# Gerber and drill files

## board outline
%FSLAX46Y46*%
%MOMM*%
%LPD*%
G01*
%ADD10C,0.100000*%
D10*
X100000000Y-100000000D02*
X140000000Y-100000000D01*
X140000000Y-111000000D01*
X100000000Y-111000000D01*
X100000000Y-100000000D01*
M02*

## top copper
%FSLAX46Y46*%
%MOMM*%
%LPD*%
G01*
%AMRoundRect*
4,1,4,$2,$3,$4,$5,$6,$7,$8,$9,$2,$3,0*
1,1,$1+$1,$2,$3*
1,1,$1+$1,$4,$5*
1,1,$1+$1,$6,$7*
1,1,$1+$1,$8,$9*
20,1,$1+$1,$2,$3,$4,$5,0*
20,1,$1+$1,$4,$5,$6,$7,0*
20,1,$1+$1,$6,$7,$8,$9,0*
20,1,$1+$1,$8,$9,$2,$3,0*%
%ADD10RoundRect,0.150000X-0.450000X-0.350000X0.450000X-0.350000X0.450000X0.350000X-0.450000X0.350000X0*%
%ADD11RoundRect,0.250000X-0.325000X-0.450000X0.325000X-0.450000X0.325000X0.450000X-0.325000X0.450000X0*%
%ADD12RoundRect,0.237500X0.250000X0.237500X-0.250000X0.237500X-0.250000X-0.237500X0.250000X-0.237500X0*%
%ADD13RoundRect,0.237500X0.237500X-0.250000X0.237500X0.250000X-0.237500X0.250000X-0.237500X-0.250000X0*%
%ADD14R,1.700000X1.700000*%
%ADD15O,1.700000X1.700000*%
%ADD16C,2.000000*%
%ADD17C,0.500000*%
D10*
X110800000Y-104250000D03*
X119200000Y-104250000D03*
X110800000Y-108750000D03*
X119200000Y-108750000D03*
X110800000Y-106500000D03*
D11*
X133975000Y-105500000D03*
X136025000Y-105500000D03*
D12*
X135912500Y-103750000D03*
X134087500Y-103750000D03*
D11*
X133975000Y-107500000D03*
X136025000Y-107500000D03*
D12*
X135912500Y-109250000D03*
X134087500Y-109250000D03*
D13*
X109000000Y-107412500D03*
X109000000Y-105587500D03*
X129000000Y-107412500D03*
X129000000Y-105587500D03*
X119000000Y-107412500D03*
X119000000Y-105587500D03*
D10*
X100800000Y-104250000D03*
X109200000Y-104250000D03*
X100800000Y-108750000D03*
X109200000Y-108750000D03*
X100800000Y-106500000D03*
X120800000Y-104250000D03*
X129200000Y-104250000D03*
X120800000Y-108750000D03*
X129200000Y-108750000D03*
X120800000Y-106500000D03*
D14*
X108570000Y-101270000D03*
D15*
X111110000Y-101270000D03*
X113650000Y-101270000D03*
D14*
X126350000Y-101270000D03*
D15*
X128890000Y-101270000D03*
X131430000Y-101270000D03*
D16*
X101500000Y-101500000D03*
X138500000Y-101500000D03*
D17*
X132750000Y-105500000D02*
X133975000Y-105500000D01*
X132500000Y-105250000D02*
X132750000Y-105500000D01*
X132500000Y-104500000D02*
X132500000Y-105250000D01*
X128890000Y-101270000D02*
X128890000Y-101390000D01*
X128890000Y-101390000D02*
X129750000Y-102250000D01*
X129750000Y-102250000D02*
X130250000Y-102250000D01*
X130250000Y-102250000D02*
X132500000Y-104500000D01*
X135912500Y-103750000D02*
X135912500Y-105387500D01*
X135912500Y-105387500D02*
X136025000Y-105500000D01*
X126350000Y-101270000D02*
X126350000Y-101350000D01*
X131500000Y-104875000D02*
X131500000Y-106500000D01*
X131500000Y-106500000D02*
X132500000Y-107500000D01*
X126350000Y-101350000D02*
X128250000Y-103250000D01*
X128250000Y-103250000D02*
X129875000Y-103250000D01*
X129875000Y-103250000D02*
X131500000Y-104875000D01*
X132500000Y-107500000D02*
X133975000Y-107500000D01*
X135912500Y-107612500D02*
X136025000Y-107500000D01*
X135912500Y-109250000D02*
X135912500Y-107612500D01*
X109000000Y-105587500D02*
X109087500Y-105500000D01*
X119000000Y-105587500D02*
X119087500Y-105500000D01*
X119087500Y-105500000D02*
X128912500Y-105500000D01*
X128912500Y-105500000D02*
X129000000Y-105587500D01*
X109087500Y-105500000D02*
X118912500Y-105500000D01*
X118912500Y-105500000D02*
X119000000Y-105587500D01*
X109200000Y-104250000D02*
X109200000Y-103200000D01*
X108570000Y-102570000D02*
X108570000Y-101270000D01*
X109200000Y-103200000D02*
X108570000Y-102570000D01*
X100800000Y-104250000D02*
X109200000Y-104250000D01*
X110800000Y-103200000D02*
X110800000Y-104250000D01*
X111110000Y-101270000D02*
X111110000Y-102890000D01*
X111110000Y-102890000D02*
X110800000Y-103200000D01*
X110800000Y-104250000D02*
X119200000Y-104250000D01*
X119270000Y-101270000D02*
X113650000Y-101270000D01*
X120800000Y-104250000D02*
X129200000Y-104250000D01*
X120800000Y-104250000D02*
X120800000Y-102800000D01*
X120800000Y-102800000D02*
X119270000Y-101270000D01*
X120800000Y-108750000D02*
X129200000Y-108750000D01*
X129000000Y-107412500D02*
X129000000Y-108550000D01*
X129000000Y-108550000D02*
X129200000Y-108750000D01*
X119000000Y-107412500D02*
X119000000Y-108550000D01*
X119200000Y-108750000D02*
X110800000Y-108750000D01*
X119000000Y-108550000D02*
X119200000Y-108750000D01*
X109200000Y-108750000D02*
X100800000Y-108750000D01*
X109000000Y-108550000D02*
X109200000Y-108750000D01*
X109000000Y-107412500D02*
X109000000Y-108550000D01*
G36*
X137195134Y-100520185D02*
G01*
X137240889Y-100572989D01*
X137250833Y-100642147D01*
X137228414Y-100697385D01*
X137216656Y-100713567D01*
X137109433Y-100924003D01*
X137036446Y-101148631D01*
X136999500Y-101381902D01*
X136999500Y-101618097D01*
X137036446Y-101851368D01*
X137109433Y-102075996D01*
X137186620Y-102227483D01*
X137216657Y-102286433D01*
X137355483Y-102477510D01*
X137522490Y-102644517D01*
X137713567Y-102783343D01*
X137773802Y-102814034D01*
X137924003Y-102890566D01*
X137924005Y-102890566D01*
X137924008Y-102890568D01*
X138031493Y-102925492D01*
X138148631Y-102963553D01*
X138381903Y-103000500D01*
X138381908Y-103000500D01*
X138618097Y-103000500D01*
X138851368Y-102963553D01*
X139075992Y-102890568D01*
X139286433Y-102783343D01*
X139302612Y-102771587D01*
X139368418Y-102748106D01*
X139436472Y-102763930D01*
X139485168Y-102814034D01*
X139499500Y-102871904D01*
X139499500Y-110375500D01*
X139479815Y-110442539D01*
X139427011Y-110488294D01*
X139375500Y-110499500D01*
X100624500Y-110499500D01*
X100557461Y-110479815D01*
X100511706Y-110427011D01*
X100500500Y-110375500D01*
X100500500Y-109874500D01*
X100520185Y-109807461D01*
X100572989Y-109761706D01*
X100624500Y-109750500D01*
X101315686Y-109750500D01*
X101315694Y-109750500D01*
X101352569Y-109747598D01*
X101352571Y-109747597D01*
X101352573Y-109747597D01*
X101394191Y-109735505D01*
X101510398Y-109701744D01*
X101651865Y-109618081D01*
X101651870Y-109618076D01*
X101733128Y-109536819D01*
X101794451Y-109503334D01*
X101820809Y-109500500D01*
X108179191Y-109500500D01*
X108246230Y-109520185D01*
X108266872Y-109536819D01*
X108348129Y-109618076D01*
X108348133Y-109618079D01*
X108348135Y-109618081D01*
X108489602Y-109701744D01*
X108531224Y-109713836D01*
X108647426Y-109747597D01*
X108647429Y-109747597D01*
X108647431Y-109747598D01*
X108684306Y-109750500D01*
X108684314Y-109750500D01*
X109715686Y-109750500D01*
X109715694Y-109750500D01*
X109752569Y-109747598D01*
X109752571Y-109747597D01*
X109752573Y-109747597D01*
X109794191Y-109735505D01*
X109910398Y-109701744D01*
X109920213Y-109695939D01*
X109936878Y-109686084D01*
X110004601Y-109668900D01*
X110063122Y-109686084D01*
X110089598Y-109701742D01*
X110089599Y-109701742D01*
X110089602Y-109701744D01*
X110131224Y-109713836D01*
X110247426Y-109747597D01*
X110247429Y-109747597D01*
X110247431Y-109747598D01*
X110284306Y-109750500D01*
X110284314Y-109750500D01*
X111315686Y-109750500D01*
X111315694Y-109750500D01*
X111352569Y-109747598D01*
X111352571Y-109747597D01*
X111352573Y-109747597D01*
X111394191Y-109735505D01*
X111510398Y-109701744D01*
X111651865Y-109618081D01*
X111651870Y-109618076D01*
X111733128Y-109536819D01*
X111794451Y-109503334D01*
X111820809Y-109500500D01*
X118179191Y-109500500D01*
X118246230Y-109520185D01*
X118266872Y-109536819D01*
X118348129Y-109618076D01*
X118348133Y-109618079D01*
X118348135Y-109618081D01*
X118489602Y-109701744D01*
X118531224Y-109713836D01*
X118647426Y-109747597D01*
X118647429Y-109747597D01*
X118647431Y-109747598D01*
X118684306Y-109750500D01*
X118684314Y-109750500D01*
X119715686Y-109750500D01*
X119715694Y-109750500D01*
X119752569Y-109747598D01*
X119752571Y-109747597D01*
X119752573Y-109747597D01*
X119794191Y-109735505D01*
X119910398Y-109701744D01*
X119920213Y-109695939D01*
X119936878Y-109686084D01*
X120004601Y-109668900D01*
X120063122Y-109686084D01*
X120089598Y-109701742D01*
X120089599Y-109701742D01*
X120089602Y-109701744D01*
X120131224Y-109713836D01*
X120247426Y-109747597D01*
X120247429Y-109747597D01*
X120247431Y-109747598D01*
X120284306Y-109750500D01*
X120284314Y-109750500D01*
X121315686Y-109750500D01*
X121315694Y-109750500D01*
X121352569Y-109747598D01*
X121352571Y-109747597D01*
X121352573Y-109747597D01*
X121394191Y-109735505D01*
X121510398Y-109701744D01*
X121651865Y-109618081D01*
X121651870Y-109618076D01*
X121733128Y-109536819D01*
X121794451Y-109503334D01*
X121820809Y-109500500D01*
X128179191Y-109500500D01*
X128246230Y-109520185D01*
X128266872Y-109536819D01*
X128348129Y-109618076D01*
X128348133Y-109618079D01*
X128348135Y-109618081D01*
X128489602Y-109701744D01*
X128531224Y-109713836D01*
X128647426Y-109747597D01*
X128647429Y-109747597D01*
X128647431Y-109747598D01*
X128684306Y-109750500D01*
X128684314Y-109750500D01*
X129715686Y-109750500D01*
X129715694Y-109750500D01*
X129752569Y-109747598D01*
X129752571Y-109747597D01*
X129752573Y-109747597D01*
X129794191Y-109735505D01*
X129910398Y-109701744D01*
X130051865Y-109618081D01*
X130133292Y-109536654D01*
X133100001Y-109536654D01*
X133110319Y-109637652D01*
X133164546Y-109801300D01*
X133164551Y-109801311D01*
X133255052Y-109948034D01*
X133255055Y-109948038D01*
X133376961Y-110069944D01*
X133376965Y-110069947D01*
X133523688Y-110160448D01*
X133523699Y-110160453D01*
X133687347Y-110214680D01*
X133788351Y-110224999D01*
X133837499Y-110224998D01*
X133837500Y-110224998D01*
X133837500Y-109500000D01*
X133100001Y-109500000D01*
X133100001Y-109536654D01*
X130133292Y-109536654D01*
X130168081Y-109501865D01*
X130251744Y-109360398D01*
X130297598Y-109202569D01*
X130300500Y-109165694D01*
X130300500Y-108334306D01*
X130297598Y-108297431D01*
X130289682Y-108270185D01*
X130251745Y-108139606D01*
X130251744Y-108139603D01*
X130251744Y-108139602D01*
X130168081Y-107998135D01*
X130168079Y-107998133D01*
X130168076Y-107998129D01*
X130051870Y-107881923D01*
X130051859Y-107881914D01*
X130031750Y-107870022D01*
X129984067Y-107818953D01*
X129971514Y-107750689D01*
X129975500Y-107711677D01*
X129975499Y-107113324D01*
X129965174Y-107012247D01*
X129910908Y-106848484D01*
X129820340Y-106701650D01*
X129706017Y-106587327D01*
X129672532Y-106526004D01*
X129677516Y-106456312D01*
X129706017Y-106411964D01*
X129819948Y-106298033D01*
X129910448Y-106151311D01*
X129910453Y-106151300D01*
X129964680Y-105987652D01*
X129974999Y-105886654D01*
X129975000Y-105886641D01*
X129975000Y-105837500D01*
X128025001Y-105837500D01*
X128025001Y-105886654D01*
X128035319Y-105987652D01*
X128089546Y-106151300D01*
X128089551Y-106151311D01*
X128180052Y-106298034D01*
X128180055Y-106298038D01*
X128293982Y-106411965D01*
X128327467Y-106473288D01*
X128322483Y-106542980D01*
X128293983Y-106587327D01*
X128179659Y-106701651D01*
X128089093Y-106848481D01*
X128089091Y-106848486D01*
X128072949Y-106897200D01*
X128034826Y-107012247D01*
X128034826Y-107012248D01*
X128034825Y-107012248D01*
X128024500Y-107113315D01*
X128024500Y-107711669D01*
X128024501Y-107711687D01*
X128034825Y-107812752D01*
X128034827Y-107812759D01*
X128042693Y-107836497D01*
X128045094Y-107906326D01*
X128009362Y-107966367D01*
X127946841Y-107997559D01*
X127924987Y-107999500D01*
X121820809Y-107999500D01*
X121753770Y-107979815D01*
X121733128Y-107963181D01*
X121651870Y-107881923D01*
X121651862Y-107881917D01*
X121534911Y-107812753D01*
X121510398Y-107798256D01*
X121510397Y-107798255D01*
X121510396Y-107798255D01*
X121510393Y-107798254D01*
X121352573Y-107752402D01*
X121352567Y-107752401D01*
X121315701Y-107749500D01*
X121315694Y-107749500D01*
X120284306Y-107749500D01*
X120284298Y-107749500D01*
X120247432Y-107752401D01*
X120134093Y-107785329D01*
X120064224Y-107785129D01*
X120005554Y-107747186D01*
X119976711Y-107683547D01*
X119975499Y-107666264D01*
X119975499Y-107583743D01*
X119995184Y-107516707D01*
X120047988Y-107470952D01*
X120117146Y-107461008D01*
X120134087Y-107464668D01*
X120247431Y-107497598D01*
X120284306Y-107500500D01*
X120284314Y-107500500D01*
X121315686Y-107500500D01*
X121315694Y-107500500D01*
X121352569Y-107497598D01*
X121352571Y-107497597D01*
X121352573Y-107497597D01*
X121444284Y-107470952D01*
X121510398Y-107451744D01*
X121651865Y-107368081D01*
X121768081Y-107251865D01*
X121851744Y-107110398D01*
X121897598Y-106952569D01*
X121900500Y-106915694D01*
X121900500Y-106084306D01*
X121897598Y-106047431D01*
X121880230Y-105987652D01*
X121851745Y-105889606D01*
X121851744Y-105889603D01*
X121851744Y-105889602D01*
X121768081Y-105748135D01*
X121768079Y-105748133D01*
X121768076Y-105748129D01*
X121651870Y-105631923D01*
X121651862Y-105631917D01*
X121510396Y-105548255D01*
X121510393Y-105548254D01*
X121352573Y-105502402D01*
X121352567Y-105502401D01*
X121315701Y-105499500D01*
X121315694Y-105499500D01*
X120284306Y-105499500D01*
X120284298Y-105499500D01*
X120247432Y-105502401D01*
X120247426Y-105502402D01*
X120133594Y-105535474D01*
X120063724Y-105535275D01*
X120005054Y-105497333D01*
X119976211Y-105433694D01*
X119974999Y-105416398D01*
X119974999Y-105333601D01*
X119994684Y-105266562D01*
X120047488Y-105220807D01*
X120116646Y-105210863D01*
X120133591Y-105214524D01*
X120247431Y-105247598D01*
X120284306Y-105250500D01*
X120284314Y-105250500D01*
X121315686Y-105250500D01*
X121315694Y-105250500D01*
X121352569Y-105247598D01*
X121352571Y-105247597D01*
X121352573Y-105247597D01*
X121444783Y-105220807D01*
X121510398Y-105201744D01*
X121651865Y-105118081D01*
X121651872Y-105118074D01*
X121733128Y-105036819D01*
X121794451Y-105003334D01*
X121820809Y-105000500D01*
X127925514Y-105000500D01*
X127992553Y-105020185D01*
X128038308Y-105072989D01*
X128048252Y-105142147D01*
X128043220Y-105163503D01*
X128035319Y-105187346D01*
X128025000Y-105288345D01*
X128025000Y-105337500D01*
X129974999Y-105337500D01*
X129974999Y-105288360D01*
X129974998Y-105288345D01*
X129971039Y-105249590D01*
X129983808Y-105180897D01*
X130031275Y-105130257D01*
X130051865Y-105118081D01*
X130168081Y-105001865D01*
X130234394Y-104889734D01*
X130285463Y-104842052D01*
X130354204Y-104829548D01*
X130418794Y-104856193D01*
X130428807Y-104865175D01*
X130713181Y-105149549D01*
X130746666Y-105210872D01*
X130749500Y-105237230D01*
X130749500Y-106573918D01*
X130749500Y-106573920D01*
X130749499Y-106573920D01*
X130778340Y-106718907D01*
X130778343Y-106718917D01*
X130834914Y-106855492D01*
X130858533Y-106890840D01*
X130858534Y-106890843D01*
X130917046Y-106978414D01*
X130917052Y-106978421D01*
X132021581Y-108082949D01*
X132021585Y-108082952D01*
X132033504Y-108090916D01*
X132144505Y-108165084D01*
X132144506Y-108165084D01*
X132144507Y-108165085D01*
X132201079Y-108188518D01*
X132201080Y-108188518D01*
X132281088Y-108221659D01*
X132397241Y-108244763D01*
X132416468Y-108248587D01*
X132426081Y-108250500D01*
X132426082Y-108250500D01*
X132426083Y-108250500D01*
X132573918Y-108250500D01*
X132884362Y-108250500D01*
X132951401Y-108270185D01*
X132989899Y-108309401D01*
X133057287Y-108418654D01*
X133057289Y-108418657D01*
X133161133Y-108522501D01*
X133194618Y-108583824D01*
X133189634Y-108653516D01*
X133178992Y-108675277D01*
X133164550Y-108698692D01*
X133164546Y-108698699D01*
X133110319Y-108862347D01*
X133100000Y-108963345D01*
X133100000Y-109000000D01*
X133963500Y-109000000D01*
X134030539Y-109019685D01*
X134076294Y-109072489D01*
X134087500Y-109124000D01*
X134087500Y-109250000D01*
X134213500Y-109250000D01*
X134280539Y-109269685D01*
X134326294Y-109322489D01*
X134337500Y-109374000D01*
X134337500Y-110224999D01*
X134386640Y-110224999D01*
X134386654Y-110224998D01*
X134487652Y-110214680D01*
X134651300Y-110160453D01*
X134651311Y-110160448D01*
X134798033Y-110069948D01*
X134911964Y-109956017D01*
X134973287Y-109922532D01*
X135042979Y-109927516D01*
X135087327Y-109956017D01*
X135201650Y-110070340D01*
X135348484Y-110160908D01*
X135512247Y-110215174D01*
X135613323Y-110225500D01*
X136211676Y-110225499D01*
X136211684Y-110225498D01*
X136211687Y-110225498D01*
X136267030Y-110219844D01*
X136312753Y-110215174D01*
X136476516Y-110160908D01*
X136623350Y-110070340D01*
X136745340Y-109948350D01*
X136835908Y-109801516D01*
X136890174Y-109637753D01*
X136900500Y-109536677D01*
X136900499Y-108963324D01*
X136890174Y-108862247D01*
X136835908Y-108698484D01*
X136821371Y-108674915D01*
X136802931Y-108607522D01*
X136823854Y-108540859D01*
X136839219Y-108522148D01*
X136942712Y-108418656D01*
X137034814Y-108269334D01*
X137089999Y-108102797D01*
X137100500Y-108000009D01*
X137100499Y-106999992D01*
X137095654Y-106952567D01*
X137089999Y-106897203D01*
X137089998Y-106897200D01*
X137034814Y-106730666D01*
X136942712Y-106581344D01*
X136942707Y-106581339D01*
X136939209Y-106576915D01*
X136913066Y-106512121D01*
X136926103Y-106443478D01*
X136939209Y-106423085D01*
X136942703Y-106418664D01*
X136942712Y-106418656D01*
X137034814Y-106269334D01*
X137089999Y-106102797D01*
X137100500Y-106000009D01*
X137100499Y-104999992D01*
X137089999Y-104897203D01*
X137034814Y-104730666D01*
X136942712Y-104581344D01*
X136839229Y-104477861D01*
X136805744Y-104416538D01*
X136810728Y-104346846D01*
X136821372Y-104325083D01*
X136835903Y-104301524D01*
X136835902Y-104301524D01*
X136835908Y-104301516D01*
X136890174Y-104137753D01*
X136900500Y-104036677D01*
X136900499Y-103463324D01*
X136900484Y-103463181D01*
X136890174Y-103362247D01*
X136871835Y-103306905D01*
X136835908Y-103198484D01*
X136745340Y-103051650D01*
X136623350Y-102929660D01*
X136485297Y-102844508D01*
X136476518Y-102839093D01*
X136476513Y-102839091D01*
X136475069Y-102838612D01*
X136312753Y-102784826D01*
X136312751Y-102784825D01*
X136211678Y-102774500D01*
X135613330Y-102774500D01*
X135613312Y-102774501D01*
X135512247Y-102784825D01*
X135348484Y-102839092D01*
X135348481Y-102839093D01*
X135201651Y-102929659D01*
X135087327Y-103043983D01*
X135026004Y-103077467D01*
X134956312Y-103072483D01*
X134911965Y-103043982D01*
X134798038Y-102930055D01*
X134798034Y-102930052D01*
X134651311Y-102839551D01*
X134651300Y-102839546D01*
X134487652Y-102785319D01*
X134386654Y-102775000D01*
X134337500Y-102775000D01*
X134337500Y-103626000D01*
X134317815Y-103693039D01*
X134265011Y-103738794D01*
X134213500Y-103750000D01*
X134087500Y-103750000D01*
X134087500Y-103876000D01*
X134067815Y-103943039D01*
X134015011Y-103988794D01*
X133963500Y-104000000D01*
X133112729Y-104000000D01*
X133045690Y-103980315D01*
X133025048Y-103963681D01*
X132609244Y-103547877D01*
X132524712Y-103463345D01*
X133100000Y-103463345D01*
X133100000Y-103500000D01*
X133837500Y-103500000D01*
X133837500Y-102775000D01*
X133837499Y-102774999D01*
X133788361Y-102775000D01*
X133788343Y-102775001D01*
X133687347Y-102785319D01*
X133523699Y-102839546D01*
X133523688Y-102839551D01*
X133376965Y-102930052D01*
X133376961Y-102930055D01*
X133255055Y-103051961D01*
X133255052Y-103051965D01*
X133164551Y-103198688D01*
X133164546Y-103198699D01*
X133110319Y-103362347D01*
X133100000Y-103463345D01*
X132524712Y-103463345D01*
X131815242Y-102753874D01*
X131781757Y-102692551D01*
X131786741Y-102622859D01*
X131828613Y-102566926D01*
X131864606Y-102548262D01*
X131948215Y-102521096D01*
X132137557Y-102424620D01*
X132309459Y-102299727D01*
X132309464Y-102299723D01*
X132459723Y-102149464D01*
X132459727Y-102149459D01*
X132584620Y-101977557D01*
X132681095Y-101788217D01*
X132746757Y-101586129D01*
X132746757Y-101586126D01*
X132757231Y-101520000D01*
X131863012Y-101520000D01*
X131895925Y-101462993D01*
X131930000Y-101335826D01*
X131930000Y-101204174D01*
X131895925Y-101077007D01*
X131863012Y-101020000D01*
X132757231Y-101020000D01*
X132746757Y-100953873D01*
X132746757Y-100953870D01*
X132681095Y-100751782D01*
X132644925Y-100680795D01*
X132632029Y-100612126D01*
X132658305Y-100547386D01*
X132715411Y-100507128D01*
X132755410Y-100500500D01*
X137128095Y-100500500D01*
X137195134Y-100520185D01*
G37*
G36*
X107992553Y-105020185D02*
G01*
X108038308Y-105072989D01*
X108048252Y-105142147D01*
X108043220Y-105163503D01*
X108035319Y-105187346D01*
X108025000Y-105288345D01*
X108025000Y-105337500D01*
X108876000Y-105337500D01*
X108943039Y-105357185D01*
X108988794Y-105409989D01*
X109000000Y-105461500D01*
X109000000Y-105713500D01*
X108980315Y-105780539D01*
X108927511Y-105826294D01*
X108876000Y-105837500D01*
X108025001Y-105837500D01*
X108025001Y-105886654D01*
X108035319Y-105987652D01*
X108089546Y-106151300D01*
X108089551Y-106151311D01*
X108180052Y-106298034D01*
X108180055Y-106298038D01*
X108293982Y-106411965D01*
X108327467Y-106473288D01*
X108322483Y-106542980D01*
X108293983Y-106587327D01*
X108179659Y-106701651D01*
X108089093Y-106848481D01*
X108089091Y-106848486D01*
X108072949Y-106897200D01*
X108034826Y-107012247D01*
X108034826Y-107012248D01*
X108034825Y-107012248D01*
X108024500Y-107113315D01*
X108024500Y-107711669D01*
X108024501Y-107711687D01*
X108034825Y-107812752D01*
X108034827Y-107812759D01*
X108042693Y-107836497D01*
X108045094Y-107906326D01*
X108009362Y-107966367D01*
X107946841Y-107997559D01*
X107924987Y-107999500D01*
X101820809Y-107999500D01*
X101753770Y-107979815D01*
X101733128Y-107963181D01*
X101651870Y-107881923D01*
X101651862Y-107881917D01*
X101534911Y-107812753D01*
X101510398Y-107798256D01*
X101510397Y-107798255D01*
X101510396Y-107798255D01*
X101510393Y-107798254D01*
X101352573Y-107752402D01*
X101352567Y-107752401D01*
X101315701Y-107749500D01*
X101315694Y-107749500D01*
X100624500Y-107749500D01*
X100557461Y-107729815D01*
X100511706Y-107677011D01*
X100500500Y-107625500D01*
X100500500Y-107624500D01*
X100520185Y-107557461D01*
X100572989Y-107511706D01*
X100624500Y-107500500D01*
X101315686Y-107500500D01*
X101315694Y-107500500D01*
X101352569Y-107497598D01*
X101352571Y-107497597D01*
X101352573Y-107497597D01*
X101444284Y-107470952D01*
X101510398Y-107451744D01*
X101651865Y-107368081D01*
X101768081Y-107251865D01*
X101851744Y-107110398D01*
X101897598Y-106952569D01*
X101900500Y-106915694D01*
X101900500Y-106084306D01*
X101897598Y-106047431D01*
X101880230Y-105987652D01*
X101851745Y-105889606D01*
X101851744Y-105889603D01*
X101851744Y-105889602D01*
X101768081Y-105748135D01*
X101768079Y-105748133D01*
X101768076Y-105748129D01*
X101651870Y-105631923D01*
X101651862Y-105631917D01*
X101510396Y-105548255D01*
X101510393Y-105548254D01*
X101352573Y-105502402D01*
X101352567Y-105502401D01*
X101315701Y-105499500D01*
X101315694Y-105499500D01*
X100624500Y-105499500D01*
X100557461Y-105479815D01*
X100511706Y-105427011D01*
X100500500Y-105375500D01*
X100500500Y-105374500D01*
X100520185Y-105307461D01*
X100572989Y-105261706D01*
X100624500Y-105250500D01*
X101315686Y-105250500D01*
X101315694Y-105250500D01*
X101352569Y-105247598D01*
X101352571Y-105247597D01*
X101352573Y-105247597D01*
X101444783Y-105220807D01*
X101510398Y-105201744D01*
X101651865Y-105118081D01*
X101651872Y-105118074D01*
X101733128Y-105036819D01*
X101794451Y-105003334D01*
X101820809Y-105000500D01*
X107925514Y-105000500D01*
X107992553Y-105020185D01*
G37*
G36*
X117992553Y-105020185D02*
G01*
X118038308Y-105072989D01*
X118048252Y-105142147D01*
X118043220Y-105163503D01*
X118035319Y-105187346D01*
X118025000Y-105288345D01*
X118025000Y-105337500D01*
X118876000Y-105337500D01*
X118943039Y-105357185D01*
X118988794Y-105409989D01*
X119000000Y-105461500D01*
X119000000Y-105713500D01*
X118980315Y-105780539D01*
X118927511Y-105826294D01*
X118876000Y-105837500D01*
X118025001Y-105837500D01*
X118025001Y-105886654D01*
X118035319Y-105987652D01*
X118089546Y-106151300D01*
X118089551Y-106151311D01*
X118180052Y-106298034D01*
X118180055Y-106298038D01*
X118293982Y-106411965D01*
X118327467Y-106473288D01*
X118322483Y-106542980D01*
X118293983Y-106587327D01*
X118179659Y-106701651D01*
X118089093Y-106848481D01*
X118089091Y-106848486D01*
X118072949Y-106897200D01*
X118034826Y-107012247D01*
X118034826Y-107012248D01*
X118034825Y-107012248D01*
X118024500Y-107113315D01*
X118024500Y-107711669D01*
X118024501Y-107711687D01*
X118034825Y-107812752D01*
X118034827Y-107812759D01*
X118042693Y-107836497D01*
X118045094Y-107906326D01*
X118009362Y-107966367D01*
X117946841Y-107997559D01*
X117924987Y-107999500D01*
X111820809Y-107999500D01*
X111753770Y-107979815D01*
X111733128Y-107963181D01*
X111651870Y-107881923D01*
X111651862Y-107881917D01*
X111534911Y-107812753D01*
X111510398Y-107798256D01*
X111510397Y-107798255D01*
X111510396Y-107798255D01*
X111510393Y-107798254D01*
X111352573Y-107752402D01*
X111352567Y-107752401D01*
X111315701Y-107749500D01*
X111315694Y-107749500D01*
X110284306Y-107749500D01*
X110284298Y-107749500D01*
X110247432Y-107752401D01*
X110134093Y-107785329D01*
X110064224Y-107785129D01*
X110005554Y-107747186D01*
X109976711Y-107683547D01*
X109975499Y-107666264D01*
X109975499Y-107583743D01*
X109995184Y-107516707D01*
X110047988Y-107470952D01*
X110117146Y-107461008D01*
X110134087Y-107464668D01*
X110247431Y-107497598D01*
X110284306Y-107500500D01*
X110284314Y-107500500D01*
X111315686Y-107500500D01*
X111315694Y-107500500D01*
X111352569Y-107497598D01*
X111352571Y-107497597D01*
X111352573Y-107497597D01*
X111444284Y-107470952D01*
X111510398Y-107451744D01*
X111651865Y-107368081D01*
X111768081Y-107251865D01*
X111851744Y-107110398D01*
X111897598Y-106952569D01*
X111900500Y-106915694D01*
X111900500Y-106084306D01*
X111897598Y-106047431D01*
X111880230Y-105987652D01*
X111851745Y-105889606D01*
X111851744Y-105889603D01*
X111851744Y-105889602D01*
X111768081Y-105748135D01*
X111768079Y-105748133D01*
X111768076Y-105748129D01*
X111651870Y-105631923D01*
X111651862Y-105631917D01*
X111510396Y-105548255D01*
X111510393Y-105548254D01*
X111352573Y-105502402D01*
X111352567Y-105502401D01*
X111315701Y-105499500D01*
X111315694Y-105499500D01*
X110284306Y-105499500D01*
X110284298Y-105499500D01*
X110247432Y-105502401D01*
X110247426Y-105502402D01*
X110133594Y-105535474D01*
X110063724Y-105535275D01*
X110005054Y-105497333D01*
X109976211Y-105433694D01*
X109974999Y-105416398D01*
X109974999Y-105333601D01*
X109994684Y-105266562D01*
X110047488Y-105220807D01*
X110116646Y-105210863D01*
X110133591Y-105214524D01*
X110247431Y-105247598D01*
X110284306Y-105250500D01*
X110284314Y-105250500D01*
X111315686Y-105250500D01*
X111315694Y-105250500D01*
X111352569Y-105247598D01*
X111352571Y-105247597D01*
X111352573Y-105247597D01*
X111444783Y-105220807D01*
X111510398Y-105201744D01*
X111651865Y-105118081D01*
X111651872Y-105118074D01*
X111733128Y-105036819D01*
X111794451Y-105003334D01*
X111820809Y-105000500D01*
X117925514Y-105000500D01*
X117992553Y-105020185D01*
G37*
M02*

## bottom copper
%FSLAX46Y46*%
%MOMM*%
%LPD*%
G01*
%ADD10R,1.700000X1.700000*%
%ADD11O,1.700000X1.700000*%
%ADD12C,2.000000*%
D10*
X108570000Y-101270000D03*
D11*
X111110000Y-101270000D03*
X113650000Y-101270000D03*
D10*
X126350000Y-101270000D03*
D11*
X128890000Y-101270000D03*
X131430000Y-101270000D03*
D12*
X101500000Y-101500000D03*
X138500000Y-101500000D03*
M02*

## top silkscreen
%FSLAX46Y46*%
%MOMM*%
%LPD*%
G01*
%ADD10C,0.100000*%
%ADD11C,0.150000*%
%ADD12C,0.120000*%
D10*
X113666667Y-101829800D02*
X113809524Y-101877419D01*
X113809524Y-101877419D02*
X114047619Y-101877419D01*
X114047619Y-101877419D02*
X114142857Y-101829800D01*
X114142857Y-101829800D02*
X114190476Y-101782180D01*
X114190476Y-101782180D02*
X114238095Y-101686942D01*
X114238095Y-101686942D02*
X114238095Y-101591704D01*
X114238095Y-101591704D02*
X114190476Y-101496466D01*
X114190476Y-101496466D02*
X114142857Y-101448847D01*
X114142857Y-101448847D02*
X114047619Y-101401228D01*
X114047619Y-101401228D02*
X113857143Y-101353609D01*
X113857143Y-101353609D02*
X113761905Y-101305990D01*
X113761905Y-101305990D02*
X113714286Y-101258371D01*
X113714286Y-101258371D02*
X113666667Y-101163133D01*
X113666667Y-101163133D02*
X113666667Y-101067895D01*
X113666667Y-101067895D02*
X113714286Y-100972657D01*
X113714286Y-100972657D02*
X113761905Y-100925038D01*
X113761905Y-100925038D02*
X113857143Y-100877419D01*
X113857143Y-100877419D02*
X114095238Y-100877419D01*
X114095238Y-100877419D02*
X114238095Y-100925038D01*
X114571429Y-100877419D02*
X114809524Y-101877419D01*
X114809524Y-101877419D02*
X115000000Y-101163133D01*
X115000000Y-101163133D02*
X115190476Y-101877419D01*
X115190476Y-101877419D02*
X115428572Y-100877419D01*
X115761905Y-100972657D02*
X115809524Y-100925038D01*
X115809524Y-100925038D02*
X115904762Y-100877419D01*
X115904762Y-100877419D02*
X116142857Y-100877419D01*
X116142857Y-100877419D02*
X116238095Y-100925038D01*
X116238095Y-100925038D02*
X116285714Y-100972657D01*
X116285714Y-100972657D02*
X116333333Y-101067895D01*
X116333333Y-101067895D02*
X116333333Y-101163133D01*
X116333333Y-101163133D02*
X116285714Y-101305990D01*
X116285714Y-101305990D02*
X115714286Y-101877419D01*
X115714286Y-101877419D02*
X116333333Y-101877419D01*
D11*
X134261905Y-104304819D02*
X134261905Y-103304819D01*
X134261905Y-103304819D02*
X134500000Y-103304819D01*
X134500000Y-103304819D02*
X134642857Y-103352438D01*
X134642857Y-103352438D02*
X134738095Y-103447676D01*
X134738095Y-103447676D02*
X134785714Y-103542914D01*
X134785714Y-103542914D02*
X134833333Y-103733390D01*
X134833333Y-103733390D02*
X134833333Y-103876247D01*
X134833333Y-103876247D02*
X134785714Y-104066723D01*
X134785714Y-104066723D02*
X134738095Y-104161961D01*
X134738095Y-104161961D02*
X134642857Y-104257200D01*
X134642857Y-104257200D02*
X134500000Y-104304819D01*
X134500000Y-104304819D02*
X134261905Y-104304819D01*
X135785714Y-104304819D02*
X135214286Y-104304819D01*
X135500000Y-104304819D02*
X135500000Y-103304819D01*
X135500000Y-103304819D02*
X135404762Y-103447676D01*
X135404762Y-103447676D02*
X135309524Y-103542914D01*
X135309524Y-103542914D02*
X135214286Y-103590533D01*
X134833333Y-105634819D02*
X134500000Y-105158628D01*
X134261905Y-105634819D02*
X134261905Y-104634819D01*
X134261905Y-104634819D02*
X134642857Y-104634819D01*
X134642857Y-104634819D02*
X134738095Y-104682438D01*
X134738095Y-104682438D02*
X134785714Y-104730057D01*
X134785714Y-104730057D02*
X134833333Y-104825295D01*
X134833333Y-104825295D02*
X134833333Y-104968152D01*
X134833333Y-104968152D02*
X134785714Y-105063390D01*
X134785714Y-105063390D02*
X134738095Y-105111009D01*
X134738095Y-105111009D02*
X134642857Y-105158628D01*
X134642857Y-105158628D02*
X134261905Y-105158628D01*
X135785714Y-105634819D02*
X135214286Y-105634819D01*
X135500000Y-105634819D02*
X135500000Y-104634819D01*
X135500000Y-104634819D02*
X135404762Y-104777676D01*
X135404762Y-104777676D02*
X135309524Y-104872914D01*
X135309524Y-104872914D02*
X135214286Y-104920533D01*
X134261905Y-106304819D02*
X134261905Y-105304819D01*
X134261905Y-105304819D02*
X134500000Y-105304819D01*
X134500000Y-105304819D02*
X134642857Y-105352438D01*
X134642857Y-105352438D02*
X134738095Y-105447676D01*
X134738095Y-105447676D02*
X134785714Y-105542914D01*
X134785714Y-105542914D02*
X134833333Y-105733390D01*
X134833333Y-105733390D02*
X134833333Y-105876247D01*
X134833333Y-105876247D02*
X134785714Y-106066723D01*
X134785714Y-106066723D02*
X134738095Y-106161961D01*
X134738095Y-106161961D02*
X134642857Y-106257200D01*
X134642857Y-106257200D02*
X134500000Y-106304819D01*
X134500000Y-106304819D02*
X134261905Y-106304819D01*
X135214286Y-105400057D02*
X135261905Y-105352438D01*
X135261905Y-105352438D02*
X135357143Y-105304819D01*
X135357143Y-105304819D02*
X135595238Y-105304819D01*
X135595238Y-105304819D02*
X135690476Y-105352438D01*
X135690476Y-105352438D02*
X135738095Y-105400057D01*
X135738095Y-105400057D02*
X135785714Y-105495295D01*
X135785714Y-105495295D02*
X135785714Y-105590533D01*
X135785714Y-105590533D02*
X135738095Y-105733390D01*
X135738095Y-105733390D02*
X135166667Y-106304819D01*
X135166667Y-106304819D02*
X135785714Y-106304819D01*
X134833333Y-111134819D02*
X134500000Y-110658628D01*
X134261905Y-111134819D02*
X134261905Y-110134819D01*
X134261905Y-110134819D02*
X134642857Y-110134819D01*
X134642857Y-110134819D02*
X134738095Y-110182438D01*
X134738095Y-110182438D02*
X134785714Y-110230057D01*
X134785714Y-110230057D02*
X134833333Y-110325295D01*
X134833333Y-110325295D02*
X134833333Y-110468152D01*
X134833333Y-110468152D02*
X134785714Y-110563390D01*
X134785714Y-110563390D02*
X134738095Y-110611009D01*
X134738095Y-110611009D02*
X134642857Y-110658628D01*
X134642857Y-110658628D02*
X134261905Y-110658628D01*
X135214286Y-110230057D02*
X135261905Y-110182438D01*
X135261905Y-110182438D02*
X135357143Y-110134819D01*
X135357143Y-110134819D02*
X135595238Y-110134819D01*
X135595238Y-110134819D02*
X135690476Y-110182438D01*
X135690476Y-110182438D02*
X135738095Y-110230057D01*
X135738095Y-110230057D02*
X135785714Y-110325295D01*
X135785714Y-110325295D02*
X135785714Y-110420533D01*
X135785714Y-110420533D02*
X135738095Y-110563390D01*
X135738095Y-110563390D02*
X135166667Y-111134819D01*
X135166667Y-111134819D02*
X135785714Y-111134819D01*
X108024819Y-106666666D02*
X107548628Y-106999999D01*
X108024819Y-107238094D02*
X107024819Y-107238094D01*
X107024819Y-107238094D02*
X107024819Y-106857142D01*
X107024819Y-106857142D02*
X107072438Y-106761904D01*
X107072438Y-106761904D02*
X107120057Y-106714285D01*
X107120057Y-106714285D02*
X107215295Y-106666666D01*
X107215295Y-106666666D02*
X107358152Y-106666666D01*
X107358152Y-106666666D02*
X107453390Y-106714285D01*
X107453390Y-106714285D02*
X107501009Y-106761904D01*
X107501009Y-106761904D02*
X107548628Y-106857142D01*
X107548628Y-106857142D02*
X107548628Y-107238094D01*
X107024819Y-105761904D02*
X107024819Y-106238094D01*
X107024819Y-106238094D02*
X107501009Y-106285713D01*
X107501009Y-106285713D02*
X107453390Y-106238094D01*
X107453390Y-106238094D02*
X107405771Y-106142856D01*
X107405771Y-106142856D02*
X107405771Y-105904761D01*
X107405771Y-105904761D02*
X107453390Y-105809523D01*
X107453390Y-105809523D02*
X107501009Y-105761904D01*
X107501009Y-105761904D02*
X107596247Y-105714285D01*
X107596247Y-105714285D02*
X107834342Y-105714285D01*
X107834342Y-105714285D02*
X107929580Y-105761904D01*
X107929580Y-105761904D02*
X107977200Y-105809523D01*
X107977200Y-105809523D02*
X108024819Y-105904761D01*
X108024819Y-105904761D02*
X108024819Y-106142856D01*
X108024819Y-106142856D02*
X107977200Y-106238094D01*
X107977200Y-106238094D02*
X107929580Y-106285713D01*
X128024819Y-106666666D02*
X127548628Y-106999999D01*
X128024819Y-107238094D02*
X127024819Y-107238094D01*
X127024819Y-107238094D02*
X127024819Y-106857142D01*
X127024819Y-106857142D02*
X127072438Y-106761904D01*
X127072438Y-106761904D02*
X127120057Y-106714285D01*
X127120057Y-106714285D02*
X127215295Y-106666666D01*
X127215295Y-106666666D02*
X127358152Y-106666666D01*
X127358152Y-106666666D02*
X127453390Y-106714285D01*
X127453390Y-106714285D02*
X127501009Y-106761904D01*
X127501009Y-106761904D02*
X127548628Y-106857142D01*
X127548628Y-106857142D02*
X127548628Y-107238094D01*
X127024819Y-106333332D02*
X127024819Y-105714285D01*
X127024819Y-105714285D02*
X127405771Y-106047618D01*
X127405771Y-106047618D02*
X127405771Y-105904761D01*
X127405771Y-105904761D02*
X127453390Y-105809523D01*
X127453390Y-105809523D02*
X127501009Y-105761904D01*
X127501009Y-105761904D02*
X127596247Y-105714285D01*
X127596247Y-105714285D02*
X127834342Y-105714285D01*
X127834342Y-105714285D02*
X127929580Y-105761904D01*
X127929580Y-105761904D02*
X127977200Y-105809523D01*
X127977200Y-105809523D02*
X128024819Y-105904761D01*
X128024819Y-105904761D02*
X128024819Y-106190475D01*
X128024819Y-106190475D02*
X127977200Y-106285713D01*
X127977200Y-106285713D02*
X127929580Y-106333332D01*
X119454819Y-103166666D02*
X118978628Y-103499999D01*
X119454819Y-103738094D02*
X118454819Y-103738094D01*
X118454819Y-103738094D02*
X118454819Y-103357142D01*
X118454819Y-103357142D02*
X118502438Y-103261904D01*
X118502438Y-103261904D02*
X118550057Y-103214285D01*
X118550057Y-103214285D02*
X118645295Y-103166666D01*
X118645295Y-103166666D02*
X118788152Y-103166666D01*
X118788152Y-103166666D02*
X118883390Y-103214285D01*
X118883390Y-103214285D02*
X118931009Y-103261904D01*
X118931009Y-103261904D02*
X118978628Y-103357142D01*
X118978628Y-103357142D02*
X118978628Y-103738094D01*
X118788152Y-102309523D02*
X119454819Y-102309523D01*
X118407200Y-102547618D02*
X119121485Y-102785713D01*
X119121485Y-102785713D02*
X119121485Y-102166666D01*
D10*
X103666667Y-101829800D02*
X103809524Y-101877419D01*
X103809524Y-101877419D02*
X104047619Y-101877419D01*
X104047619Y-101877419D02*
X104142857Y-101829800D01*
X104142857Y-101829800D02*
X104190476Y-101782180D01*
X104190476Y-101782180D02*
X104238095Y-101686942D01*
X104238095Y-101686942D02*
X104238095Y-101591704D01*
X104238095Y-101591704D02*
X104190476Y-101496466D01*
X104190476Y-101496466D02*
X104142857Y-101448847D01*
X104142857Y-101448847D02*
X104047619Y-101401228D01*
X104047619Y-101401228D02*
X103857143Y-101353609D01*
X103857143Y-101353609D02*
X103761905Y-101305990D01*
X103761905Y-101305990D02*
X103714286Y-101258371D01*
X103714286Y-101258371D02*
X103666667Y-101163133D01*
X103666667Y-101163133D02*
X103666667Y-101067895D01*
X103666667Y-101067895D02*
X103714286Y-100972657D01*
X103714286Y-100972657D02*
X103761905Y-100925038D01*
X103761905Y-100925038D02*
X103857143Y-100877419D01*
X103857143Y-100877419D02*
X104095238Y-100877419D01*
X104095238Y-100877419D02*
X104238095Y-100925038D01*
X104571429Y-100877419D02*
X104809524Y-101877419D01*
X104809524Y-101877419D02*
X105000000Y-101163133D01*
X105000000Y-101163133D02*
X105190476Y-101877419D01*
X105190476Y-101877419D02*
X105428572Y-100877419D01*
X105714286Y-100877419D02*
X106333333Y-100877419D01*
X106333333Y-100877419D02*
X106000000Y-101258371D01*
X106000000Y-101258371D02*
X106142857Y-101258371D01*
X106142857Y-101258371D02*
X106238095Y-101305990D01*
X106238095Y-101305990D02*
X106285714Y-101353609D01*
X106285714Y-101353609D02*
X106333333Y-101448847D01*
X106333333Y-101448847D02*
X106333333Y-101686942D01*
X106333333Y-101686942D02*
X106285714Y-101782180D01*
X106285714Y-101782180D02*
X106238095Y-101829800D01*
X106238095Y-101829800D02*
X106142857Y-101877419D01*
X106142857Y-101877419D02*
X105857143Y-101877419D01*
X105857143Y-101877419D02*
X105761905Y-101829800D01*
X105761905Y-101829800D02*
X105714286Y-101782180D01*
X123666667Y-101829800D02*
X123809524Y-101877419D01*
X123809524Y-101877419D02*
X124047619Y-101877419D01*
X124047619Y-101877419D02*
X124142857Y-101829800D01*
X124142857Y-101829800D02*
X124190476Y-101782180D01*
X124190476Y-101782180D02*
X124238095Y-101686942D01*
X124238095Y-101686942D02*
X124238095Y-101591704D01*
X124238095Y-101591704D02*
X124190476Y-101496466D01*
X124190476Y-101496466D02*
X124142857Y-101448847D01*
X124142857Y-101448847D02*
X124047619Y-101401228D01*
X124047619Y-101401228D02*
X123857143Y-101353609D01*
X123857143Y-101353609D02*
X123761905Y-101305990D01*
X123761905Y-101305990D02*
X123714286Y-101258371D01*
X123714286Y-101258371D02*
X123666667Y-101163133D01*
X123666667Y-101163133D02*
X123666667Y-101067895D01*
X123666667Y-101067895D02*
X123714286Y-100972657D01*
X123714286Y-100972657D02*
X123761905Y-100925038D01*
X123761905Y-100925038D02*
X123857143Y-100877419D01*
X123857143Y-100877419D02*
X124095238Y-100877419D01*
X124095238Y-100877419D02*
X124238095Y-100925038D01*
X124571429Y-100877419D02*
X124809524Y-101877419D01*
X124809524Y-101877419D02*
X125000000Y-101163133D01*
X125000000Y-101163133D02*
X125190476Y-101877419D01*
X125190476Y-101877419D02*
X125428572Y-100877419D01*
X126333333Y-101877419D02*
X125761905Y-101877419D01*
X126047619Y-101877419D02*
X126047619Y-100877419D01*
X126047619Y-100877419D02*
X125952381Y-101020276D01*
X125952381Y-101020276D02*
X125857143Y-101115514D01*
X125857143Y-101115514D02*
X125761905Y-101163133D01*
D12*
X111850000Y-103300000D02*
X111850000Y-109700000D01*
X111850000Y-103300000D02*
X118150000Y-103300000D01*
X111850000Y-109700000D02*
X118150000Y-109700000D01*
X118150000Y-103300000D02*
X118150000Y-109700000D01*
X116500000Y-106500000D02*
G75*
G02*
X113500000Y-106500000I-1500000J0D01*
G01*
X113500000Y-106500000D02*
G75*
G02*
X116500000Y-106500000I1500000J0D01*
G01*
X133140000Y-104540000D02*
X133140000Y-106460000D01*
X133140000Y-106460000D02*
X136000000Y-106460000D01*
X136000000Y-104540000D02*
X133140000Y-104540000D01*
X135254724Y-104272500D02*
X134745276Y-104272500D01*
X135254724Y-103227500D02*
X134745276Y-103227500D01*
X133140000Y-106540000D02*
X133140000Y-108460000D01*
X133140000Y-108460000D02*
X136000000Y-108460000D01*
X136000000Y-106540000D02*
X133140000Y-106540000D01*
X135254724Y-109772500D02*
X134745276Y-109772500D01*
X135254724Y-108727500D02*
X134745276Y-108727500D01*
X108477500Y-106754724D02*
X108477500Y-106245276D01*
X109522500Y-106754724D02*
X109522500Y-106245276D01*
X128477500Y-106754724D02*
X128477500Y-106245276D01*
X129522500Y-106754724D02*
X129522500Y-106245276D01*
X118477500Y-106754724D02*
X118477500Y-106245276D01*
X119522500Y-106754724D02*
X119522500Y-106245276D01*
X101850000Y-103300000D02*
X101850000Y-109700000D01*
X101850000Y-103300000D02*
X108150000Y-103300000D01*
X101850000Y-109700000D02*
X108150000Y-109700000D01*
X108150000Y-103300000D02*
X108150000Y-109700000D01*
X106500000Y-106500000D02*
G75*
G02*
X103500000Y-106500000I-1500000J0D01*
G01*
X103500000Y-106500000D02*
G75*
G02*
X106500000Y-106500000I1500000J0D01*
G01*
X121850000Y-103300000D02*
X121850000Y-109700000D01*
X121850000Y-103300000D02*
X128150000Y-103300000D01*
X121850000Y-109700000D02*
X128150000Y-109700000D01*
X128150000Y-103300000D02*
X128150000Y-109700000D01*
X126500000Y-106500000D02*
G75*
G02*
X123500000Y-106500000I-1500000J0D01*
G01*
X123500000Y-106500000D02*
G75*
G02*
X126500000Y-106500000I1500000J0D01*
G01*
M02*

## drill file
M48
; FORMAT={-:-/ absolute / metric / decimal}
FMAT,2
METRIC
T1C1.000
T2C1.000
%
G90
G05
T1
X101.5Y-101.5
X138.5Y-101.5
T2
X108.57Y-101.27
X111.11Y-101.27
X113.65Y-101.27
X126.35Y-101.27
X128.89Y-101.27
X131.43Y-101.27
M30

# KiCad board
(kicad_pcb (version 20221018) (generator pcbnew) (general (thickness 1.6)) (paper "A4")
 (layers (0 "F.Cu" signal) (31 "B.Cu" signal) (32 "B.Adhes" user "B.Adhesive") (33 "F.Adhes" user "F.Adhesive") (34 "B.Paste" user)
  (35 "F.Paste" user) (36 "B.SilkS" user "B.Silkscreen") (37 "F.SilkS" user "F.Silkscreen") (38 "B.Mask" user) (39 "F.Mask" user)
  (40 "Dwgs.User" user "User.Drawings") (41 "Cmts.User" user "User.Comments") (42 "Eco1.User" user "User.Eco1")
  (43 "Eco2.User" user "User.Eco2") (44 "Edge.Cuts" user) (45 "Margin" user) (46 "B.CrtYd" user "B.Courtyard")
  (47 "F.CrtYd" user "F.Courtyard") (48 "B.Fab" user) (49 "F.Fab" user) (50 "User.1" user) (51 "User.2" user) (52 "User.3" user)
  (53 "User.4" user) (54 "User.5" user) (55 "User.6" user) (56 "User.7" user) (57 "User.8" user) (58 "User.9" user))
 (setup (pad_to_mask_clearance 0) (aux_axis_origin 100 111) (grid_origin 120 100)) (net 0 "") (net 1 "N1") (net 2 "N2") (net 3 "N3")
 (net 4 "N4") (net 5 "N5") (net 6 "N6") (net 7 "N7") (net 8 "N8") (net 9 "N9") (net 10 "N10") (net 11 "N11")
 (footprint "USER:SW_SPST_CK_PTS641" (layer "F.Cu") (at 115 106.5)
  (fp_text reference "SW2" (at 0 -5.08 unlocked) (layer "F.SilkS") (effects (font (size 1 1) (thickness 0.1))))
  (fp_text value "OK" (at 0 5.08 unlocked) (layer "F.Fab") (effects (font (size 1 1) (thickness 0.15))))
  (fp_line (start -3.15 -3.2) (end -3.15 3.2) (stroke (width 0.12) (type default)) (layer "F.SilkS"))
  (fp_line (start -3.15 -3.2) (end 3.15 -3.2) (stroke (width 0.12) (type solid)) (layer "F.SilkS"))
  (fp_line (start -3.15 3.2) (end 3.15 3.2) (stroke (width 0.12) (type solid)) (layer "F.SilkS"))
  (fp_line (start 3.15 -3.2) (end 3.15 3.2) (stroke (width 0.12) (type solid)) (layer "F.SilkS"))
  (fp_circle (center 0 0) (end 1.5 0) (stroke (width 0.12) (type default)) (fill none) (layer "F.SilkS"))
  (pad "1" smd roundrect (at -4.2 -2.25) (size 1.2 1) (layers "F.Cu" "F.Paste" "F.Mask") (roundrect_rratio 0.15) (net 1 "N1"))
  (pad "1" smd roundrect (at 4.2 -2.25) (size 1.2 1) (layers "F.Cu" "F.Paste" "F.Mask") (roundrect_rratio 0.15) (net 1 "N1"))
  (pad "2" smd roundrect (at -4.2 2.25) (size 1.2 1) (layers "F.Cu" "F.Paste" "F.Mask") (roundrect_rratio 0.15) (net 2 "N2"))
  (pad "2" smd roundrect (at 4.2 2.25) (size 1.2 1) (layers "F.Cu" "F.Paste" "F.Mask") (roundrect_rratio 0.15) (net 2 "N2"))
  (pad "SH" smd roundrect (at -4.2 0) (size 1.2 1) (layers "F.Cu" "F.Paste" "F.Mask") (roundrect_rratio 0.15)))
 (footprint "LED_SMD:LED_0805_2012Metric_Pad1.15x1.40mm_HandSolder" (layer "F.Cu") (at 135 105.5)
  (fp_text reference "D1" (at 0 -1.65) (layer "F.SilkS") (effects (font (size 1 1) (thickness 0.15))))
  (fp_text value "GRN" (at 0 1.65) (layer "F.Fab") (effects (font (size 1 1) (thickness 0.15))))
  (fp_line (start -1.86 -0.96) (end -1.86 0.96) (stroke (width 0.12) (type solid)) (layer "F.SilkS"))
  (fp_line (start -1.86 0.96) (end 1 0.96) (stroke (width 0.12) (type solid)) (layer "F.SilkS"))
  (fp_line (start 1 -0.96) (end -1.86 -0.96) (stroke (width 0.12) (type solid)) (layer "F.SilkS"))
  (pad "1" smd roundrect (at -1.025 0) (size 1.15 1.4) (layers "F.Cu" "F.Paste" "F.Mask") (roundrect_rratio 0.2173913043) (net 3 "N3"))
  (pad "2" smd roundrect (at 1.025 0) (size 1.15 1.4) (layers "F.Cu" "F.Paste" "F.Mask") (roundrect_rratio 0.2173913043) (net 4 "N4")))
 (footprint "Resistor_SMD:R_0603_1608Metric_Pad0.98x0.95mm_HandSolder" (layer "F.Cu") (at 135 103.75 180)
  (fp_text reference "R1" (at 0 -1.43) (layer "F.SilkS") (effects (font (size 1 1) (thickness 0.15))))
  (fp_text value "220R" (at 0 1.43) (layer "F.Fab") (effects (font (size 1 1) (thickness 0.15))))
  (fp_line (start -0.254724 -0.5225) (end 0.254724 -0.5225) (stroke (width 0.12) (type solid)) (layer "F.SilkS"))
  (fp_line (start -0.254724 0.5225) (end 0.254724 0.5225) (stroke (width 0.12) (type solid)) (layer "F.SilkS"))
  (pad "1" smd roundrect (at -0.9125 0 180) (size 0.975 0.95) (layers "F.Cu" "F.Paste" "F.Mask") (roundrect_rratio 0.25) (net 4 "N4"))
  (pad "2" smd roundrect (at 0.9125 0 180) (size 0.975 0.95) (layers "F.Cu" "F.Paste" "F.Mask") (roundrect_rratio 0.25) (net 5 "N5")))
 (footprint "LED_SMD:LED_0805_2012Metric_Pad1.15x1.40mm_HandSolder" (layer "F.Cu") (at 135 107.5)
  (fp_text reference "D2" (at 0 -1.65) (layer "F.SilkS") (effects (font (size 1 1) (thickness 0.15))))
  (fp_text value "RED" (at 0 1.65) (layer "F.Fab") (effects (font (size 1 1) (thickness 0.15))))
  (fp_line (start -1.86 -0.96) (end -1.86 0.96) (stroke (width 0.12) (type solid)) (layer "F.SilkS"))
  (fp_line (start -1.86 0.96) (end 1 0.96) (stroke (width 0.12) (type solid)) (layer "F.SilkS"))
  (fp_line (start 1 -0.96) (end -1.86 -0.96) (stroke (width 0.12) (type solid)) (layer "F.SilkS"))
  (pad "1" smd roundrect (at -1.025 0) (size 1.15 1.4) (layers "F.Cu" "F.Paste" "F.Mask") (roundrect_rratio 0.2173913043) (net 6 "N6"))
  (pad "2" smd roundrect (at 1.025 0) (size 1.15 1.4) (layers "F.Cu" "F.Paste" "F.Mask") (roundrect_rratio 0.2173913043) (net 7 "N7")))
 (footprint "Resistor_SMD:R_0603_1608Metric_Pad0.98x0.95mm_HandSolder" (layer "F.Cu") (at 135 109.25 180)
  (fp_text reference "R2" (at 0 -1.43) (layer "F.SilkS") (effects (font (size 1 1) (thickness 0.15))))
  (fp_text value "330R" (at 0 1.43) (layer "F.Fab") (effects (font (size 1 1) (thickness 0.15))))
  (fp_line (start -0.254724 -0.5225) (end 0.254724 -0.5225) (stroke (width 0.12) (type solid)) (layer "F.SilkS"))
  (fp_line (start -0.254724 0.5225) (end 0.254724 0.5225) (stroke (width 0.12) (type solid)) (layer "F.SilkS"))
  (pad "1" smd roundrect (at -0.9125 0 180) (size 0.975 0.95) (layers "F.Cu" "F.Paste" "F.Mask") (roundrect_rratio 0.25) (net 7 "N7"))
  (pad "2" smd roundrect (at 0.9125 0 180) (size 0.975 0.95) (layers "F.Cu" "F.Paste" "F.Mask") (roundrect_rratio 0.25) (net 5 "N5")))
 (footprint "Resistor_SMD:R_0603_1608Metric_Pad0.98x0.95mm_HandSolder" (layer "F.Cu") (at 109 106.5 90)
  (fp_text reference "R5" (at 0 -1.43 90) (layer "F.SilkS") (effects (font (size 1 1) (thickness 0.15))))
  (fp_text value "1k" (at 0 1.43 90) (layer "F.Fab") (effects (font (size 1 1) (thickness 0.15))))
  (fp_line (start -0.254724 -0.5225) (end 0.254724 -0.5225) (stroke (width 0.12) (type solid)) (layer "F.SilkS"))
  (fp_line (start -0.254724 0.5225) (end 0.254724 0.5225) (stroke (width 0.12) (type solid)) (layer "F.SilkS"))
  (pad "1" smd roundrect (at -0.9125 0 90) (size 0.975 0.95) (layers "F.Cu" "F.Paste" "F.Mask") (roundrect_rratio 0.25) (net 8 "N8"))
  (pad "2" smd roundrect (at 0.9125 0 90) (size 0.975 0.95) (layers "F.Cu" "F.Paste" "F.Mask") (roundrect_rratio 0.25) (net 5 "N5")))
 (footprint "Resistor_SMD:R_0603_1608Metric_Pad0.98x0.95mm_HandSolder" (layer "F.Cu") (at 129 106.5 90)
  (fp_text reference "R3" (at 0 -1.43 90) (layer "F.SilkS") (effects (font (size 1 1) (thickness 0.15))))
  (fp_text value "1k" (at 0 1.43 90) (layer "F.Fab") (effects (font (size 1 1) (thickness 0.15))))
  (fp_line (start -0.254724 -0.5225) (end 0.254724 -0.5225) (stroke (width 0.12) (type solid)) (layer "F.SilkS"))
  (fp_line (start -0.254724 0.5225) (end 0.254724 0.5225) (stroke (width 0.12) (type solid)) (layer "F.SilkS"))
  (pad "1" smd roundrect (at -0.9125 0 90) (size 0.975 0.95) (layers "F.Cu" "F.Paste" "F.Mask") (roundrect_rratio 0.25) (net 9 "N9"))
  (pad "2" smd roundrect (at 0.9125 0 90) (size 0.975 0.95) (layers "F.Cu" "F.Paste" "F.Mask") (roundrect_rratio 0.25) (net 5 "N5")))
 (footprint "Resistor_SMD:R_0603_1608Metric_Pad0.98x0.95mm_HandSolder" (layer "F.Cu") (at 119 106.5 90)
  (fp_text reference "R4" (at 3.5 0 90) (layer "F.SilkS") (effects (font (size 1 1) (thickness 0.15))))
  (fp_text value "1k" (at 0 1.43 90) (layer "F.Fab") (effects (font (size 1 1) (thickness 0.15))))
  (fp_line (start -0.254724 -0.5225) (end 0.254724 -0.5225) (stroke (width 0.12) (type solid)) (layer "F.SilkS"))
  (fp_line (start -0.254724 0.5225) (end 0.254724 0.5225) (stroke (width 0.12) (type solid)) (layer "F.SilkS"))
  (pad "1" smd roundrect (at -0.9125 0 90) (size 0.975 0.95) (layers "F.Cu" "F.Paste" "F.Mask") (roundrect_rratio 0.25) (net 2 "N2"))
  (pad "2" smd roundrect (at 0.9125 0 90) (size 0.975 0.95) (layers "F.Cu" "F.Paste" "F.Mask") (roundrect_rratio 0.25) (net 5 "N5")))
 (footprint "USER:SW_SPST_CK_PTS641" (layer "F.Cu") (at 105 106.5)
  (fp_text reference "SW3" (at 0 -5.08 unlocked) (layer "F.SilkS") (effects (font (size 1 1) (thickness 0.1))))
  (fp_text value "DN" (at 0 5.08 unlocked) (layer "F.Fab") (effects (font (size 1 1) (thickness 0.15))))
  (fp_line (start -3.15 -3.2) (end -3.15 3.2) (stroke (width 0.12) (type default)) (layer "F.SilkS"))
  (fp_line (start -3.15 -3.2) (end 3.15 -3.2) (stroke (width 0.12) (type solid)) (layer "F.SilkS"))
  (fp_line (start -3.15 3.2) (end 3.15 3.2) (stroke (width 0.12) (type solid)) (layer "F.SilkS"))
  (fp_line (start 3.15 -3.2) (end 3.15 3.2) (stroke (width 0.12) (type solid)) (layer "F.SilkS"))
  (fp_circle (center 0 0) (end 1.5 0) (stroke (width 0.12) (type default)) (fill none) (layer "F.SilkS"))
  (pad "1" smd roundrect (at -4.2 -2.25) (size 1.2 1) (layers "F.Cu" "F.Paste" "F.Mask") (roundrect_rratio 0.15) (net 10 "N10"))
  (pad "1" smd roundrect (at 4.2 -2.25) (size 1.2 1) (layers "F.Cu" "F.Paste" "F.Mask") (roundrect_rratio 0.15) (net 10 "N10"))
  (pad "2" smd roundrect (at -4.2 2.25) (size 1.2 1) (layers "F.Cu" "F.Paste" "F.Mask") (roundrect_rratio 0.15) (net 8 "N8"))
  (pad "2" smd roundrect (at 4.2 2.25) (size 1.2 1) (layers "F.Cu" "F.Paste" "F.Mask") (roundrect_rratio 0.15) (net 8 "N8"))
  (pad "SH" smd roundrect (at -4.2 0) (size 1.2 1) (layers "F.Cu" "F.Paste" "F.Mask") (roundrect_rratio 0.15)))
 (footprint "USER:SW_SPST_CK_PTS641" (layer "F.Cu") (at 125 106.5)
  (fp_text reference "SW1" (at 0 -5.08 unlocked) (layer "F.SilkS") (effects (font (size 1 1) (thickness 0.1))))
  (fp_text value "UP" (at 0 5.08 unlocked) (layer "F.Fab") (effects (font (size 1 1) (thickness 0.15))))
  (fp_line (start -3.15 -3.2) (end -3.15 3.2) (stroke (width 0.12) (type default)) (layer "F.SilkS"))
  (fp_line (start -3.15 -3.2) (end 3.15 -3.2) (stroke (width 0.12) (type solid)) (layer "F.SilkS"))
  (fp_line (start -3.15 3.2) (end 3.15 3.2) (stroke (width 0.12) (type solid)) (layer "F.SilkS"))
  (fp_line (start 3.15 -3.2) (end 3.15 3.2) (stroke (width 0.12) (type solid)) (layer "F.SilkS"))
  (fp_circle (center 0 0) (end 1.5 0) (stroke (width 0.12) (type default)) (fill none) (layer "F.SilkS"))
  (pad "1" smd roundrect (at -4.2 -2.25) (size 1.2 1) (layers "F.Cu" "F.Paste" "F.Mask") (roundrect_rratio 0.15) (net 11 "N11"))
  (pad "1" smd roundrect (at 4.2 -2.25) (size 1.2 1) (layers "F.Cu" "F.Paste" "F.Mask") (roundrect_rratio 0.15) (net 11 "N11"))
  (pad "2" smd roundrect (at -4.2 2.25) (size 1.2 1) (layers "F.Cu" "F.Paste" "F.Mask") (roundrect_rratio 0.15) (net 9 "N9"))
  (pad "2" smd roundrect (at 4.2 2.25) (size 1.2 1) (layers "F.Cu" "F.Paste" "F.Mask") (roundrect_rratio 0.15) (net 9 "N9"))
  (pad "SH" smd roundrect (at -4.2 0) (size 1.2 1) (layers "F.Cu" "F.Paste" "F.Mask") (roundrect_rratio 0.15)))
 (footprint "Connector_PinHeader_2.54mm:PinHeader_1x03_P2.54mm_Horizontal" (layer "B.Cu") (at 108.57 101.27 -90)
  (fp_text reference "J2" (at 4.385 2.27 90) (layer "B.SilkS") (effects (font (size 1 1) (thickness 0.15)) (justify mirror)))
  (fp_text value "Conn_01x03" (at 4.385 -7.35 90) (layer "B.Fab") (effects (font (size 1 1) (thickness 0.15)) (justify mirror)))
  (pad "1" thru_hole rect (at 0 0 270) (size 1.7 1.7) (drill 1) (layers "*.Cu" "*.Mask") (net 10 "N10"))
  (pad "2" thru_hole oval (at 0 -2.54 270) (size 1.7 1.7) (drill 1) (layers "*.Cu" "*.Mask") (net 1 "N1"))
  (pad "3" thru_hole oval (at 0 -5.08 270) (size 1.7 1.7) (drill 1) (layers "*.Cu" "*.Mask") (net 11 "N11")))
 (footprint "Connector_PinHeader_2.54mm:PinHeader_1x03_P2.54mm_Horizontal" (layer "B.Cu") (at 126.35 101.27 -90)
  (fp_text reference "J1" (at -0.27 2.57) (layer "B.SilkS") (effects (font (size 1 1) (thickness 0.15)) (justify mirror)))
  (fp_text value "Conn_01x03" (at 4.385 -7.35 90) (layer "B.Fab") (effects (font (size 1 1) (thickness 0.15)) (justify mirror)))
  (pad "1" thru_hole rect (at 0 0 270) (size 1.7 1.7) (drill 1) (layers "*.Cu" "*.Mask") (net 6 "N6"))
  (pad "2" thru_hole oval (at 0 -2.54 270) (size 1.7 1.7) (drill 1) (layers "*.Cu" "*.Mask") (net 3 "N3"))
  (pad "3" thru_hole oval (at 0 -5.08 270) (size 1.7 1.7) (drill 1) (layers "*.Cu" "*.Mask") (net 5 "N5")))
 (gr_rect (start 100 100) (end 140 111) (stroke (width 0.1) (type default)) (fill none) (layer "Edge.Cuts"))
 (via (at 101.5 101.5) (size 2) (drill 1) (layers "F.Cu" "B.Cu") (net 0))
 (via (at 138.5 101.5) (size 2) (drill 1) (layers "F.Cu" "B.Cu") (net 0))
 (segment (start 132.75 105.5) (end 133.975 105.5) (width 0.5) (layer "F.Cu") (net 3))
 (segment (start 132.5 105.25) (end 132.75 105.5) (width 0.5) (layer "F.Cu") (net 3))
 (segment (start 132.5 104.5) (end 132.5 105.25) (width 0.5) (layer "F.Cu") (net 3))
 (segment (start 128.89 101.27) (end 128.89 101.39) (width 0.5) (layer "F.Cu") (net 3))
 (segment (start 128.89 101.39) (end 129.75 102.25) (width 0.5) (layer "F.Cu") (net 3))
 (segment (start 129.75 102.25) (end 130.25 102.25) (width 0.5) (layer "F.Cu") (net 3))
 (segment (start 130.25 102.25) (end 132.5 104.5) (width 0.5) (layer "F.Cu") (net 3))
 (segment (start 135.9125 103.75) (end 135.9125 105.3875) (width 0.5) (layer "F.Cu") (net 4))
 (segment (start 135.9125 105.3875) (end 136.025 105.5) (width 0.5) (layer "F.Cu") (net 4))
 (segment (start 126.35 101.27) (end 126.35 101.35) (width 0.5) (layer "F.Cu") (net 6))
 (segment (start 131.5 104.875) (end 131.5 106.5) (width 0.5) (layer "F.Cu") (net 6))
 (segment (start 131.5 106.5) (end 132.5 107.5) (width 0.5) (layer "F.Cu") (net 6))
 (segment (start 126.35 101.35) (end 128.25 103.25) (width 0.5) (layer "F.Cu") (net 6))
 (segment (start 128.25 103.25) (end 129.875 103.25) (width 0.5) (layer "F.Cu") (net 6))
 (segment (start 129.875 103.25) (end 131.5 104.875) (width 0.5) (layer "F.Cu") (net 6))
 (segment (start 132.5 107.5) (end 133.975 107.5) (width 0.5) (layer "F.Cu") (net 6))
 (segment (start 135.9125 107.6125) (end 136.025 107.5) (width 0.5) (layer "F.Cu") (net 7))
 (segment (start 135.9125 109.25) (end 135.9125 107.6125) (width 0.5) (layer "F.Cu") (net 7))
 (segment (start 109 105.5875) (end 109.0875 105.5) (width 0.5) (layer "F.Cu") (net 5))
 (segment (start 119 105.5875) (end 119.0875 105.5) (width 0.5) (layer "F.Cu") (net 5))
 (segment (start 119.0875 105.5) (end 128.9125 105.5) (width 0.5) (layer "F.Cu") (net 5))
 (segment (start 128.9125 105.5) (end 129 105.5875) (width 0.5) (layer "F.Cu") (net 5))
 (segment (start 109.0875 105.5) (end 118.9125 105.5) (width 0.5) (layer "F.Cu") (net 5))
 (segment (start 118.9125 105.5) (end 119 105.5875) (width 0.5) (layer "F.Cu") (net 5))
 (segment (start 109.2 104.25) (end 109.2 103.2) (width 0.5) (layer "F.Cu") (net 10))
 (segment (start 108.57 102.57) (end 108.57 101.27) (width 0.5) (layer "F.Cu") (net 10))
 (segment (start 109.2 103.2) (end 108.57 102.57) (width 0.5) (layer "F.Cu") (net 10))
 (segment (start 100.8 104.25) (end 109.2 104.25) (width 0.5) (layer "F.Cu") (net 10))
 (segment (start 110.8 103.2) (end 110.8 104.25) (width 0.5) (layer "F.Cu") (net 1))
 (segment (start 111.11 101.27) (end 111.11 102.89) (width 0.5) (layer "F.Cu") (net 1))
 (segment (start 111.11 102.89) (end 110.8 103.2) (width 0.5) (layer "F.Cu") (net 1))
 (segment (start 110.8 104.25) (end 119.2 104.25) (width 0.5) (layer "F.Cu") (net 1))
 (segment (start 119.27 101.27) (end 113.65 101.27) (width 0.5) (layer "F.Cu") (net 11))
 (segment (start 120.8 104.25) (end 129.2 104.25) (width 0.5) (layer "F.Cu") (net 11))
 (segment (start 120.8 104.25) (end 120.8 102.8) (width 0.5) (layer "F.Cu") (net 11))
 (segment (start 120.8 102.8) (end 119.27 101.27) (width 0.5) (layer "F.Cu") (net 11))
 (segment (start 120.8 108.75) (end 129.2 108.75) (width 0.5) (layer "F.Cu") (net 9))
 (segment (start 129 107.4125) (end 129 108.55) (width 0.5) (layer "F.Cu") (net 9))
 (segment (start 129 108.55) (end 129.2 108.75) (width 0.5) (layer "F.Cu") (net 9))
 (segment (start 119 107.4125) (end 119 108.55) (width 0.5) (layer "F.Cu") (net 2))
 (segment (start 119.2 108.75) (end 110.8 108.75) (width 0.5) (layer "F.Cu") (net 2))
 (segment (start 119 108.55) (end 119.2 108.75) (width 0.5) (layer "F.Cu") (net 2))
 (segment (start 109.2 108.75) (end 100.8 108.75) (width 0.5) (layer "F.Cu") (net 8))
 (segment (start 109 108.55) (end 109.2 108.75) (width 0.5) (layer "F.Cu") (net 8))
 (segment (start 109 107.4125) (end 109 108.55) (width 0.5) (layer "F.Cu") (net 8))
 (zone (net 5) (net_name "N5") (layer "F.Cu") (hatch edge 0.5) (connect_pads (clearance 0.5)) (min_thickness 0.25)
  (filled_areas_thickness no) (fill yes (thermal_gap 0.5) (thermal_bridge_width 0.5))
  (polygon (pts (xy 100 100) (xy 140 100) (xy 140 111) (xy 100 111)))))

